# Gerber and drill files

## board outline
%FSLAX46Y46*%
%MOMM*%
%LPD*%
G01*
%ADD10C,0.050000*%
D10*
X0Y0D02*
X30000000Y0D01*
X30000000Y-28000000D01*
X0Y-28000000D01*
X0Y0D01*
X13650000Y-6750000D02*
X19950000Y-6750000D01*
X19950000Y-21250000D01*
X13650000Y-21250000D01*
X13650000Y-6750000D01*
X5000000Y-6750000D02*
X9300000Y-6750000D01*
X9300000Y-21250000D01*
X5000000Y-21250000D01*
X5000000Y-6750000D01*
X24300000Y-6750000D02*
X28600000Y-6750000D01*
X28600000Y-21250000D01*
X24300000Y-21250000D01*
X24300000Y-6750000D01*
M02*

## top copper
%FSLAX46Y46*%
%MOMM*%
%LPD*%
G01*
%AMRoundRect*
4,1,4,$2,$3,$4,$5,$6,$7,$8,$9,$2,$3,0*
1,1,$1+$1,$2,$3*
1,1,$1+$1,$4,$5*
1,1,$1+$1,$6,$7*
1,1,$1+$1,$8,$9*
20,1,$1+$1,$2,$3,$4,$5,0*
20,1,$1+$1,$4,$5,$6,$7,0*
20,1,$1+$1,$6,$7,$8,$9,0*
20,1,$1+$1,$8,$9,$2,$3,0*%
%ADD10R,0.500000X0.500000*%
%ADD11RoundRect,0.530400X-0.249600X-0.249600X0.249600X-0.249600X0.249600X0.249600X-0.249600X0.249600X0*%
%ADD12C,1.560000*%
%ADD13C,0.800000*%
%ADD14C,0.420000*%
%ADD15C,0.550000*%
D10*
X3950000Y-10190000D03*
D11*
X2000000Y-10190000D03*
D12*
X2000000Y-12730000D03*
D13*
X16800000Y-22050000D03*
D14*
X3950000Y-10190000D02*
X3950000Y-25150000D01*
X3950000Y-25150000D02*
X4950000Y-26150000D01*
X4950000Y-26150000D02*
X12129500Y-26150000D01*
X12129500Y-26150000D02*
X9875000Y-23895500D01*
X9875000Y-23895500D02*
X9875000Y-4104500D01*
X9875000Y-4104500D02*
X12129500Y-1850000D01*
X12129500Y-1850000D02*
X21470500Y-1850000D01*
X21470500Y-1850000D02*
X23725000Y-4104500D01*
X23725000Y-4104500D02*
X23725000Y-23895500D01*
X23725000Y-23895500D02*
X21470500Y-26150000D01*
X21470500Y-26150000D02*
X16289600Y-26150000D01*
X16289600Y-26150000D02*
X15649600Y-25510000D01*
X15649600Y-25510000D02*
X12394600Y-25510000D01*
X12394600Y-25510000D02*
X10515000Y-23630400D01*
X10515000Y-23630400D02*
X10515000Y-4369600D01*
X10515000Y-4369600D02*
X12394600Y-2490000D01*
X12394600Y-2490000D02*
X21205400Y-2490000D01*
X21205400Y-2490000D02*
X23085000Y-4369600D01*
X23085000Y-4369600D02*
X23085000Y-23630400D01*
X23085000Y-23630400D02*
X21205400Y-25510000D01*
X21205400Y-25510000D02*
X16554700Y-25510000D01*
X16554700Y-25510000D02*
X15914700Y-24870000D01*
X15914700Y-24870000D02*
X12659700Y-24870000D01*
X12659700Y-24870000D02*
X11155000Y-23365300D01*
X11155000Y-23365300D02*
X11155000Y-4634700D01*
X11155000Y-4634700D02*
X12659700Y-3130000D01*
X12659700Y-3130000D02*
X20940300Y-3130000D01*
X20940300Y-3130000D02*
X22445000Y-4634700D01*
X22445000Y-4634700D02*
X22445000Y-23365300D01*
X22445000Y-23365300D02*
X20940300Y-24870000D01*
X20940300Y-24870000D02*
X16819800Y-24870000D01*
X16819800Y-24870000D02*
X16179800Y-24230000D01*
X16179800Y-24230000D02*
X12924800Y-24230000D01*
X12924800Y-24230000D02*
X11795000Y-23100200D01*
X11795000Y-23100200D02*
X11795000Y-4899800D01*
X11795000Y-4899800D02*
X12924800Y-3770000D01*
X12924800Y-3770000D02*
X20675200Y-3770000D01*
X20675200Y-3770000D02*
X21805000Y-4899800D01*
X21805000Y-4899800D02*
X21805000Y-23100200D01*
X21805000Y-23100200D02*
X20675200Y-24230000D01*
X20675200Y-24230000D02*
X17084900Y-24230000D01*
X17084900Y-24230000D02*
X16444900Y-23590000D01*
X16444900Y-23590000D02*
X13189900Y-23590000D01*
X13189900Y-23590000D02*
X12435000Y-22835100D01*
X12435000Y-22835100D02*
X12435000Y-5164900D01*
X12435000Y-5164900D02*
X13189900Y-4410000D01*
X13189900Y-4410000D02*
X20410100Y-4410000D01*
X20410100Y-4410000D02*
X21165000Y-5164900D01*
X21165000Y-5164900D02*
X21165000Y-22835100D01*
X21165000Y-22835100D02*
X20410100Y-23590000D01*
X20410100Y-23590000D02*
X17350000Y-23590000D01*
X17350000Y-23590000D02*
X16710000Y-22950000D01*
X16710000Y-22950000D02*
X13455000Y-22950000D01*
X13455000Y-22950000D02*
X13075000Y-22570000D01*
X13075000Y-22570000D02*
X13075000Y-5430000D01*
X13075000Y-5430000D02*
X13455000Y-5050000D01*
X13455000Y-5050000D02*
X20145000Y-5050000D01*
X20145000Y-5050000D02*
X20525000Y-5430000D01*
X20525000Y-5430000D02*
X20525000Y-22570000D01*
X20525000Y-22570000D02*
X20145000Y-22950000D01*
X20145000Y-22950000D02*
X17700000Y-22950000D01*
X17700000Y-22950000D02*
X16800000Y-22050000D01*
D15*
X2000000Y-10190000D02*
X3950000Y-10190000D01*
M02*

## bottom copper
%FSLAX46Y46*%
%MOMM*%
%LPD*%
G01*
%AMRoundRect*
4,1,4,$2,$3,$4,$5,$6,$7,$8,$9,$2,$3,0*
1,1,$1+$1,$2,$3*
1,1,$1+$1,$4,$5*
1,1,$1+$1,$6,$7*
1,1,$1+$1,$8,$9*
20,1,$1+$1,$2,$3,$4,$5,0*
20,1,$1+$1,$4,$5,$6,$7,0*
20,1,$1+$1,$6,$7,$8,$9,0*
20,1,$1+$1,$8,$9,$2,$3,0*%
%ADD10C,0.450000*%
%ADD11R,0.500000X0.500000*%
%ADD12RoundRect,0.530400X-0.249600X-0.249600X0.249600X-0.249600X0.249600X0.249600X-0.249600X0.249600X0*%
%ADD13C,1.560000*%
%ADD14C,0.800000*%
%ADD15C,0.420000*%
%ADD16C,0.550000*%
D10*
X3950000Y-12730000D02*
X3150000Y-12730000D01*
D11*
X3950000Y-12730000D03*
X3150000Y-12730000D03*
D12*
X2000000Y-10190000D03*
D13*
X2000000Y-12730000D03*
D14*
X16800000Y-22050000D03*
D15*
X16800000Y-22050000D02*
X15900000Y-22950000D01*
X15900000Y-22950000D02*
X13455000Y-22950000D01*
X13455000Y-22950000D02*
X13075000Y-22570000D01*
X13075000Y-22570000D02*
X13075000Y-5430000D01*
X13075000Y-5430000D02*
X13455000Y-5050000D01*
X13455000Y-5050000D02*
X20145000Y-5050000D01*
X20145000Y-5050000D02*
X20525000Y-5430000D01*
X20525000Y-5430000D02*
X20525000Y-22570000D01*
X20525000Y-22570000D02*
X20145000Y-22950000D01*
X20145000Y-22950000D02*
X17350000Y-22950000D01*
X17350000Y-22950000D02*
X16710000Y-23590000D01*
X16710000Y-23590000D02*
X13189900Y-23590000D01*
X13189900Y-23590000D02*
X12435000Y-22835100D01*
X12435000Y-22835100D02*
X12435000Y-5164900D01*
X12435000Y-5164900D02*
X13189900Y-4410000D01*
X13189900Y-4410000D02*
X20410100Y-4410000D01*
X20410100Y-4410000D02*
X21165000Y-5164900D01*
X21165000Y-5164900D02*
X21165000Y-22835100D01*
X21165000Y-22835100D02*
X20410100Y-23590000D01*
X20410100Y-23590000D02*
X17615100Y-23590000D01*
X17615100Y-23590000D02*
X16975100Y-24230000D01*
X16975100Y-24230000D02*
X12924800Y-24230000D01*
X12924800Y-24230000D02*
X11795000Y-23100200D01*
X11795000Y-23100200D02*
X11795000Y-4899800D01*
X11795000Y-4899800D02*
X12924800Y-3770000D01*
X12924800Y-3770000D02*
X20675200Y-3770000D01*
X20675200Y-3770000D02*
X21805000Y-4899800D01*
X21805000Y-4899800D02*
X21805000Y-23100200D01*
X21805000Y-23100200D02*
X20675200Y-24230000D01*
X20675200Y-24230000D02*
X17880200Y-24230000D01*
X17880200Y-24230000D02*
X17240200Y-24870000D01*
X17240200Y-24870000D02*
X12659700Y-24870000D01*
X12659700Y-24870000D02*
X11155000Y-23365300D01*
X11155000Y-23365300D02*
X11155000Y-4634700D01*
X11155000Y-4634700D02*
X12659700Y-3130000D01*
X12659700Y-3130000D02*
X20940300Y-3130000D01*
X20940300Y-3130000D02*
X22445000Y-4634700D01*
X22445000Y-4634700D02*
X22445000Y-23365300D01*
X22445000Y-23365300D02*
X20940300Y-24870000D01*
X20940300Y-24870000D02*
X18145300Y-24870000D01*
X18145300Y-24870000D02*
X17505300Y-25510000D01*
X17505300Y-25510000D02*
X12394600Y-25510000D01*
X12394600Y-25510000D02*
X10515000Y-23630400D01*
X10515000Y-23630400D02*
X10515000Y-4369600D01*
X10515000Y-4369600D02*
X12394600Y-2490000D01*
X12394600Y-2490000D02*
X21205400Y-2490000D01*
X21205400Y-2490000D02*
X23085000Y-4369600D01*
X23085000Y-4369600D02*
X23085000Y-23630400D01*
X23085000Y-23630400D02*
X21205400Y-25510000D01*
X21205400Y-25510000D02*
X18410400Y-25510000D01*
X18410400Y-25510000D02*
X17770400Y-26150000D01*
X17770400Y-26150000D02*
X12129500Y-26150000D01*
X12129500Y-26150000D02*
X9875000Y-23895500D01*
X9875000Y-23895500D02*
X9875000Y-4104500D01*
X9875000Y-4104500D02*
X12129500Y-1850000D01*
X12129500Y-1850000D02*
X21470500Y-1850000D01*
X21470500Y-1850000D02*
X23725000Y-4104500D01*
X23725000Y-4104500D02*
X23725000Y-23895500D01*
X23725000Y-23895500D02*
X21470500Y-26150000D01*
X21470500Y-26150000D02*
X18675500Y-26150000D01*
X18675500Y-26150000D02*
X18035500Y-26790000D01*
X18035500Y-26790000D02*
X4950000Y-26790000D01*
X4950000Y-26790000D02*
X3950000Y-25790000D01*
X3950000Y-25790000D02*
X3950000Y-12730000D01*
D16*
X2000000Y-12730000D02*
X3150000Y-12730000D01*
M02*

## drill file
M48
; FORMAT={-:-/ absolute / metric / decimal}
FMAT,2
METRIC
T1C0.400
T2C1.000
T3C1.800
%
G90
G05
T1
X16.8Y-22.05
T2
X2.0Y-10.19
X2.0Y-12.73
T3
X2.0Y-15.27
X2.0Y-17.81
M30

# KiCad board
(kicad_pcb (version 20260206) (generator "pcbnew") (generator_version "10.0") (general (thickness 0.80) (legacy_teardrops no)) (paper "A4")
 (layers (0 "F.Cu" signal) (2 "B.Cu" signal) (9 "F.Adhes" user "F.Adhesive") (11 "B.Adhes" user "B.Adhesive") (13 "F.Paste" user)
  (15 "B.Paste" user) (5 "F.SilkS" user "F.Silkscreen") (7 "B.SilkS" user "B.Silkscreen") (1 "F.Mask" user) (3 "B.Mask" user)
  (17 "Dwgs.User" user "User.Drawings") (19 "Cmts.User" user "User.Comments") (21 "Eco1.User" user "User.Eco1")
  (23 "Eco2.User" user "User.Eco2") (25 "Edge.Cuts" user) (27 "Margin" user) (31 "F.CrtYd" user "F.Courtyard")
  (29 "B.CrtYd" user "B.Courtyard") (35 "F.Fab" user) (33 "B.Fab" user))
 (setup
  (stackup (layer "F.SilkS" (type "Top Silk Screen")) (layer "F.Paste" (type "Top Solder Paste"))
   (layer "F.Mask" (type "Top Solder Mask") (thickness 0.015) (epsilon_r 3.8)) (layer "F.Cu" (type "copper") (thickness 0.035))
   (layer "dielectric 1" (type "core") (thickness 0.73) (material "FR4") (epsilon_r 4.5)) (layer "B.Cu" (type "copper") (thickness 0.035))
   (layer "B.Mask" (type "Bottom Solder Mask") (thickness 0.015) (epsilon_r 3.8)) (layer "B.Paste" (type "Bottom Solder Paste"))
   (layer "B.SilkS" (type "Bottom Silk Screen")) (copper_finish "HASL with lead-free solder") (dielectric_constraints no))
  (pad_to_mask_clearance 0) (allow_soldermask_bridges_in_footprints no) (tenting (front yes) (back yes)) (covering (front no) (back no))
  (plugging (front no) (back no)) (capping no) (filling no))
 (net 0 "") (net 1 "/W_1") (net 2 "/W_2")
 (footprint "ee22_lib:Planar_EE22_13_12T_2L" (layer "F.Cu") (at 16.8000 14.0000)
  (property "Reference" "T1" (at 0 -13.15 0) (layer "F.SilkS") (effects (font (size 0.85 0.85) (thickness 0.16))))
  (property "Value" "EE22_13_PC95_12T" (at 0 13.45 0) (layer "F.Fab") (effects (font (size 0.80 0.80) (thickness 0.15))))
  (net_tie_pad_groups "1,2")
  (fp_line (start -12.85 -1.27) (end -13.65 -1.27) (stroke (width 0.45) (type solid)) (layer "B.Cu"))
  (pad "1" smd rect (at -12.85 -3.81) (size 0.50 0.50) (layers "F.Cu") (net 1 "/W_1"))
  (pad "1" smd rect (at -12.85 -1.27) (size 0.50 0.50) (layers "B.Cu") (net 1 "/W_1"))
  (pad "2" smd rect (at -13.65 -1.27) (size 0.50 0.50) (layers "B.Cu") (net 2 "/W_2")))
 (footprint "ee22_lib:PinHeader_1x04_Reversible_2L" (layer "F.Cu") (at 2.0000 14.0000)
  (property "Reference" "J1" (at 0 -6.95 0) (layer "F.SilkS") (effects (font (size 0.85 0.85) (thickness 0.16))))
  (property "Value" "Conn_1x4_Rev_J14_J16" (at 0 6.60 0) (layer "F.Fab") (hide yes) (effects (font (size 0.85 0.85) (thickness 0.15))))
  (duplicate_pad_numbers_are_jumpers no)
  (pad "1" thru_hole roundrect (at 0 -3.81) (size 1.56 1.56) (drill 1.00) (layers "*.Cu" "*.Mask") (roundrect_rratio 0.34)
   (remove_unused_layers no) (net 1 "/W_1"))
  (pad "2" thru_hole circle (at 0 -1.27) (size 1.56 1.56) (drill 1.00) (layers "*.Cu" "*.Mask") (remove_unused_layers no) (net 2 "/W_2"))
  (pad "" np_thru_hole circle (at 0 1.27) (size 1.80 1.80) (drill 1.80) (layers "*.Cu" "*.Mask"))
  (pad "" np_thru_hole circle (at 0 3.81) (size 1.80 1.80) (drill 1.80) (layers "*.Cu" "*.Mask")))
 (gr_rect (start 0.0000 0.0000) (end 30.0000 28.0000) (stroke (width 0.05) (type solid)) (fill none) (layer "Edge.Cuts"))
 (gr_rect (start 13.6500 6.7500) (end 19.9500 21.2500) (stroke (width 0.05) (type solid)) (fill none) (layer "Edge.Cuts"))
 (gr_rect (start 5.0000 6.7500) (end 9.3000 21.2500) (stroke (width 0.05) (type solid)) (fill none) (layer "Edge.Cuts"))
 (gr_rect (start 24.3000 6.7500) (end 28.6000 21.2500) (stroke (width 0.05) (type solid)) (fill none) (layer "Edge.Cuts"))
 (via (at 16.8000 22.0500) (size 0.80) (drill 0.40) (layers "F.Cu" "B.Cu") (remove_unused_layers no) (keep_end_layers yes) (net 1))
 (segment (start 3.9500 10.1900) (end 3.9500 25.1500) (width 0.4200) (layer "F.Cu") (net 1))
 (segment (start 3.9500 25.1500) (end 4.9500 26.1500) (width 0.4200) (layer "F.Cu") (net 1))
 (segment (start 4.9500 26.1500) (end 12.1295 26.1500) (width 0.4200) (layer "F.Cu") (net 1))
 (segment (start 12.1295 26.1500) (end 9.8750 23.8955) (width 0.4200) (layer "F.Cu") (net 1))
 (segment (start 9.8750 23.8955) (end 9.8750 4.1045) (width 0.4200) (layer "F.Cu") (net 1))
 (segment (start 9.8750 4.1045) (end 12.1295 1.8500) (width 0.4200) (layer "F.Cu") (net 1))
 (segment (start 12.1295 1.8500) (end 21.4705 1.8500) (width 0.4200) (layer "F.Cu") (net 1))
 (segment (start 21.4705 1.8500) (end 23.7250 4.1045) (width 0.4200) (layer "F.Cu") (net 1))
 (segment (start 23.7250 4.1045) (end 23.7250 23.8955) (width 0.4200) (layer "F.Cu") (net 1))
 (segment (start 23.7250 23.8955) (end 21.4705 26.1500) (width 0.4200) (layer "F.Cu") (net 1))
 (segment (start 21.4705 26.1500) (end 16.2896 26.1500) (width 0.4200) (layer "F.Cu") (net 1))
 (segment (start 16.2896 26.1500) (end 15.6496 25.5100) (width 0.4200) (layer "F.Cu") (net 1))
 (segment (start 15.6496 25.5100) (end 12.3946 25.5100) (width 0.4200) (layer "F.Cu") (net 1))
 (segment (start 12.3946 25.5100) (end 10.5150 23.6304) (width 0.4200) (layer "F.Cu") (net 1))
 (segment (start 10.5150 23.6304) (end 10.5150 4.3696) (width 0.4200) (layer "F.Cu") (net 1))
 (segment (start 10.5150 4.3696) (end 12.3946 2.4900) (width 0.4200) (layer "F.Cu") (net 1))
 (segment (start 12.3946 2.4900) (end 21.2054 2.4900) (width 0.4200) (layer "F.Cu") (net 1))
 (segment (start 21.2054 2.4900) (end 23.0850 4.3696) (width 0.4200) (layer "F.Cu") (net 1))
 (segment (start 23.0850 4.3696) (end 23.0850 23.6304) (width 0.4200) (layer "F.Cu") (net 1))
 (segment (start 23.0850 23.6304) (end 21.2054 25.5100) (width 0.4200) (layer "F.Cu") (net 1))
 (segment (start 21.2054 25.5100) (end 16.5547 25.5100) (width 0.4200) (layer "F.Cu") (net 1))
 (segment (start 16.5547 25.5100) (end 15.9147 24.8700) (width 0.4200) (layer "F.Cu") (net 1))
 (segment (start 15.9147 24.8700) (end 12.6597 24.8700) (width 0.4200) (layer "F.Cu") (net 1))
 (segment (start 12.6597 24.8700) (end 11.1550 23.3653) (width 0.4200) (layer "F.Cu") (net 1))
 (segment (start 11.1550 23.3653) (end 11.1550 4.6347) (width 0.4200) (layer "F.Cu") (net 1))
 (segment (start 11.1550 4.6347) (end 12.6597 3.1300) (width 0.4200) (layer "F.Cu") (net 1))
 (segment (start 12.6597 3.1300) (end 20.9403 3.1300) (width 0.4200) (layer "F.Cu") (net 1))
 (segment (start 20.9403 3.1300) (end 22.4450 4.6347) (width 0.4200) (layer "F.Cu") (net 1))
 (segment (start 22.4450 4.6347) (end 22.4450 23.3653) (width 0.4200) (layer "F.Cu") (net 1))
 (segment (start 22.4450 23.3653) (end 20.9403 24.8700) (width 0.4200) (layer "F.Cu") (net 1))
 (segment (start 20.9403 24.8700) (end 16.8198 24.8700) (width 0.4200) (layer "F.Cu") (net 1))
 (segment (start 16.8198 24.8700) (end 16.1798 24.2300) (width 0.4200) (layer "F.Cu") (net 1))
 (segment (start 16.1798 24.2300) (end 12.9248 24.2300) (width 0.4200) (layer "F.Cu") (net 1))
 (segment (start 12.9248 24.2300) (end 11.7950 23.1002) (width 0.4200) (layer "F.Cu") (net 1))
 (segment (start 11.7950 23.1002) (end 11.7950 4.8998) (width 0.4200) (layer "F.Cu") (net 1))
 (segment (start 11.7950 4.8998) (end 12.9248 3.7700) (width 0.4200) (layer "F.Cu") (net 1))
 (segment (start 12.9248 3.7700) (end 20.6752 3.7700) (width 0.4200) (layer "F.Cu") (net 1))
 (segment (start 20.6752 3.7700) (end 21.8050 4.8998) (width 0.4200) (layer "F.Cu") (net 1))
 (segment (start 21.8050 4.8998) (end 21.8050 23.1002) (width 0.4200) (layer "F.Cu") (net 1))
 (segment (start 21.8050 23.1002) (end 20.6752 24.2300) (width 0.4200) (layer "F.Cu") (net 1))
 (segment (start 20.6752 24.2300) (end 17.0849 24.2300) (width 0.4200) (layer "F.Cu") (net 1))
 (segment (start 17.0849 24.2300) (end 16.4449 23.5900) (width 0.4200) (layer "F.Cu") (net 1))
 (segment (start 16.4449 23.5900) (end 13.1899 23.5900) (width 0.4200) (layer "F.Cu") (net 1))
 (segment (start 13.1899 23.5900) (end 12.4350 22.8351) (width 0.4200) (layer "F.Cu") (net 1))
 (segment (start 12.4350 22.8351) (end 12.4350 5.1649) (width 0.4200) (layer "F.Cu") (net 1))
 (segment (start 12.4350 5.1649) (end 13.1899 4.4100) (width 0.4200) (layer "F.Cu") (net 1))
 (segment (start 13.1899 4.4100) (end 20.4101 4.4100) (width 0.4200) (layer "F.Cu") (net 1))
 (segment (start 20.4101 4.4100) (end 21.1650 5.1649) (width 0.4200) (layer "F.Cu") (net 1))
 (segment (start 21.1650 5.1649) (end 21.1650 22.8351) (width 0.4200) (layer "F.Cu") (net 1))
 (segment (start 21.1650 22.8351) (end 20.4101 23.5900) (width 0.4200) (layer "F.Cu") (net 1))
 (segment (start 20.4101 23.5900) (end 17.3500 23.5900) (width 0.4200) (layer "F.Cu") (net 1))
 (segment (start 17.3500 23.5900) (end 16.7100 22.9500) (width 0.4200) (layer "F.Cu") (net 1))
 (segment (start 16.7100 22.9500) (end 13.4550 22.9500) (width 0.4200) (layer "F.Cu") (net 1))
 (segment (start 13.4550 22.9500) (end 13.0750 22.5700) (width 0.4200) (layer "F.Cu") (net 1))
 (segment (start 13.0750 22.5700) (end 13.0750 5.4300) (width 0.4200) (layer "F.Cu") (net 1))
 (segment (start 13.0750 5.4300) (end 13.4550 5.0500) (width 0.4200) (layer "F.Cu") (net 1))
 (segment (start 13.4550 5.0500) (end 20.1450 5.0500) (width 0.4200) (layer "F.Cu") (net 1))
 (segment (start 20.1450 5.0500) (end 20.5250 5.4300) (width 0.4200) (layer "F.Cu") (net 1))
 (segment (start 20.5250 5.4300) (end 20.5250 22.5700) (width 0.4200) (layer "F.Cu") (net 1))
 (segment (start 20.5250 22.5700) (end 20.1450 22.9500) (width 0.4200) (layer "F.Cu") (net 1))
 (segment (start 20.1450 22.9500) (end 17.7000 22.9500) (width 0.4200) (layer "F.Cu") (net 1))
 (segment (start 17.7000 22.9500) (end 16.8000 22.0500) (width 0.4200) (layer "F.Cu") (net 1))
 (segment (start 16.8000 22.0500) (end 15.9000 22.9500) (width 0.4200) (layer "B.Cu") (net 1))
 (segment (start 15.9000 22.9500) (end 13.4550 22.9500) (width 0.4200) (layer "B.Cu") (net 1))
 (segment (start 13.4550 22.9500) (end 13.0750 22.5700) (width 0.4200) (layer "B.Cu") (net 1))
 (segment (start 13.0750 22.5700) (end 13.0750 5.4300) (width 0.4200) (layer "B.Cu") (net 1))
 (segment (start 13.0750 5.4300) (end 13.4550 5.0500) (width 0.4200) (layer "B.Cu") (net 1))
 (segment (start 13.4550 5.0500) (end 20.1450 5.0500) (width 0.4200) (layer "B.Cu") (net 1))
 (segment (start 20.1450 5.0500) (end 20.5250 5.4300) (width 0.4200) (layer "B.Cu") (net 1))
 (segment (start 20.5250 5.4300) (end 20.5250 22.5700) (width 0.4200) (layer "B.Cu") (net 1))
 (segment (start 20.5250 22.5700) (end 20.1450 22.9500) (width 0.4200) (layer "B.Cu") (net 1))
 (segment (start 20.1450 22.9500) (end 17.3500 22.9500) (width 0.4200) (layer "B.Cu") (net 1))
 (segment (start 17.3500 22.9500) (end 16.7100 23.5900) (width 0.4200) (layer "B.Cu") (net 1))
 (segment (start 16.7100 23.5900) (end 13.1899 23.5900) (width 0.4200) (layer "B.Cu") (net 1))
 (segment (start 13.1899 23.5900) (end 12.4350 22.8351) (width 0.4200) (layer "B.Cu") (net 1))
 (segment (start 12.4350 22.8351) (end 12.4350 5.1649) (width 0.4200) (layer "B.Cu") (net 1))
 (segment (start 12.4350 5.1649) (end 13.1899 4.4100) (width 0.4200) (layer "B.Cu") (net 1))
 (segment (start 13.1899 4.4100) (end 20.4101 4.4100) (width 0.4200) (layer "B.Cu") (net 1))
 (segment (start 20.4101 4.4100) (end 21.1650 5.1649) (width 0.4200) (layer "B.Cu") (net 1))
 (segment (start 21.1650 5.1649) (end 21.1650 22.8351) (width 0.4200) (layer "B.Cu") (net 1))
 (segment (start 21.1650 22.8351) (end 20.4101 23.5900) (width 0.4200) (layer "B.Cu") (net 1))
 (segment (start 20.4101 23.5900) (end 17.6151 23.5900) (width 0.4200) (layer "B.Cu") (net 1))
 (segment (start 17.6151 23.5900) (end 16.9751 24.2300) (width 0.4200) (layer "B.Cu") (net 1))
 (segment (start 16.9751 24.2300) (end 12.9248 24.2300) (width 0.4200) (layer "B.Cu") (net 1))
 (segment (start 12.9248 24.2300) (end 11.7950 23.1002) (width 0.4200) (layer "B.Cu") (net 1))
 (segment (start 11.7950 23.1002) (end 11.7950 4.8998) (width 0.4200) (layer "B.Cu") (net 1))
 (segment (start 11.7950 4.8998) (end 12.9248 3.7700) (width 0.4200) (layer "B.Cu") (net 1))
 (segment (start 12.9248 3.7700) (end 20.6752 3.7700) (width 0.4200) (layer "B.Cu") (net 1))
 (segment (start 20.6752 3.7700) (end 21.8050 4.8998) (width 0.4200) (layer "B.Cu") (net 1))
 (segment (start 21.8050 4.8998) (end 21.8050 23.1002) (width 0.4200) (layer "B.Cu") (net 1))
 (segment (start 21.8050 23.1002) (end 20.6752 24.2300) (width 0.4200) (layer "B.Cu") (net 1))
 (segment (start 20.6752 24.2300) (end 17.8802 24.2300) (width 0.4200) (layer "B.Cu") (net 1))
 (segment (start 17.8802 24.2300) (end 17.2402 24.8700) (width 0.4200) (layer "B.Cu") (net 1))
 (segment (start 17.2402 24.8700) (end 12.6597 24.8700) (width 0.4200) (layer "B.Cu") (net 1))
 (segment (start 12.6597 24.8700) (end 11.1550 23.3653) (width 0.4200) (layer "B.Cu") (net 1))
 (segment (start 11.1550 23.3653) (end 11.1550 4.6347) (width 0.4200) (layer "B.Cu") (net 1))
 (segment (start 11.1550 4.6347) (end 12.6597 3.1300) (width 0.4200) (layer "B.Cu") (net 1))
 (segment (start 12.6597 3.1300) (end 20.9403 3.1300) (width 0.4200) (layer "B.Cu") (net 1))
 (segment (start 20.9403 3.1300) (end 22.4450 4.6347) (width 0.4200) (layer "B.Cu") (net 1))
 (segment (start 22.4450 4.6347) (end 22.4450 23.3653) (width 0.4200) (layer "B.Cu") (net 1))
 (segment (start 22.4450 23.3653) (end 20.9403 24.8700) (width 0.4200) (layer "B.Cu") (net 1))
 (segment (start 20.9403 24.8700) (end 18.1453 24.8700) (width 0.4200) (layer "B.Cu") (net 1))
 (segment (start 18.1453 24.8700) (end 17.5053 25.5100) (width 0.4200) (layer "B.Cu") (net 1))
 (segment (start 17.5053 25.5100) (end 12.3946 25.5100) (width 0.4200) (layer "B.Cu") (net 1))
 (segment (start 12.3946 25.5100) (end 10.5150 23.6304) (width 0.4200) (layer "B.Cu") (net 1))
 (segment (start 10.5150 23.6304) (end 10.5150 4.3696) (width 0.4200) (layer "B.Cu") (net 1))
 (segment (start 10.5150 4.3696) (end 12.3946 2.4900) (width 0.4200) (layer "B.Cu") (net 1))
 (segment (start 12.3946 2.4900) (end 21.2054 2.4900) (width 0.4200) (layer "B.Cu") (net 1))
 (segment (start 21.2054 2.4900) (end 23.0850 4.3696) (width 0.4200) (layer "B.Cu") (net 1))
 (segment (start 23.0850 4.3696) (end 23.0850 23.6304) (width 0.4200) (layer "B.Cu") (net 1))
 (segment (start 23.0850 23.6304) (end 21.2054 25.5100) (width 0.4200) (layer "B.Cu") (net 1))
 (segment (start 21.2054 25.5100) (end 18.4104 25.5100) (width 0.4200) (layer "B.Cu") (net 1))
 (segment (start 18.4104 25.5100) (end 17.7704 26.1500) (width 0.4200) (layer "B.Cu") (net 1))
 (segment (start 17.7704 26.1500) (end 12.1295 26.1500) (width 0.4200) (layer "B.Cu") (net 1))
 (segment (start 12.1295 26.1500) (end 9.8750 23.8955) (width 0.4200) (layer "B.Cu") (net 1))
 (segment (start 9.8750 23.8955) (end 9.8750 4.1045) (width 0.4200) (layer "B.Cu") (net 1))
 (segment (start 9.8750 4.1045) (end 12.1295 1.8500) (width 0.4200) (layer "B.Cu") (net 1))
 (segment (start 12.1295 1.8500) (end 21.4705 1.8500) (width 0.4200) (layer "B.Cu") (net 1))
 (segment (start 21.4705 1.8500) (end 23.7250 4.1045) (width 0.4200) (layer "B.Cu") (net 1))
 (segment (start 23.7250 4.1045) (end 23.7250 23.8955) (width 0.4200) (layer "B.Cu") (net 1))
 (segment (start 23.7250 23.8955) (end 21.4705 26.1500) (width 0.4200) (layer "B.Cu") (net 1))
 (segment (start 21.4705 26.1500) (end 18.6755 26.1500) (width 0.4200) (layer "B.Cu") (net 1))
 (segment (start 18.6755 26.1500) (end 18.0355 26.7900) (width 0.4200) (layer "B.Cu") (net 1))
 (segment (start 18.0355 26.7900) (end 4.9500 26.7900) (width 0.4200) (layer "B.Cu") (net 1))
 (segment (start 4.9500 26.7900) (end 3.9500 25.7900) (width 0.4200) (layer "B.Cu") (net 1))
 (segment (start 3.9500 25.7900) (end 3.9500 12.7300) (width 0.4200) (layer "B.Cu") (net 1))
 (segment (start 2.0000 10.1900) (end 3.9500 10.1900) (width 0.5500) (layer "F.Cu") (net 1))
 (segment (start 2.0000 12.7300) (end 3.1500 12.7300) (width 0.5500) (layer "B.Cu") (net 2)))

